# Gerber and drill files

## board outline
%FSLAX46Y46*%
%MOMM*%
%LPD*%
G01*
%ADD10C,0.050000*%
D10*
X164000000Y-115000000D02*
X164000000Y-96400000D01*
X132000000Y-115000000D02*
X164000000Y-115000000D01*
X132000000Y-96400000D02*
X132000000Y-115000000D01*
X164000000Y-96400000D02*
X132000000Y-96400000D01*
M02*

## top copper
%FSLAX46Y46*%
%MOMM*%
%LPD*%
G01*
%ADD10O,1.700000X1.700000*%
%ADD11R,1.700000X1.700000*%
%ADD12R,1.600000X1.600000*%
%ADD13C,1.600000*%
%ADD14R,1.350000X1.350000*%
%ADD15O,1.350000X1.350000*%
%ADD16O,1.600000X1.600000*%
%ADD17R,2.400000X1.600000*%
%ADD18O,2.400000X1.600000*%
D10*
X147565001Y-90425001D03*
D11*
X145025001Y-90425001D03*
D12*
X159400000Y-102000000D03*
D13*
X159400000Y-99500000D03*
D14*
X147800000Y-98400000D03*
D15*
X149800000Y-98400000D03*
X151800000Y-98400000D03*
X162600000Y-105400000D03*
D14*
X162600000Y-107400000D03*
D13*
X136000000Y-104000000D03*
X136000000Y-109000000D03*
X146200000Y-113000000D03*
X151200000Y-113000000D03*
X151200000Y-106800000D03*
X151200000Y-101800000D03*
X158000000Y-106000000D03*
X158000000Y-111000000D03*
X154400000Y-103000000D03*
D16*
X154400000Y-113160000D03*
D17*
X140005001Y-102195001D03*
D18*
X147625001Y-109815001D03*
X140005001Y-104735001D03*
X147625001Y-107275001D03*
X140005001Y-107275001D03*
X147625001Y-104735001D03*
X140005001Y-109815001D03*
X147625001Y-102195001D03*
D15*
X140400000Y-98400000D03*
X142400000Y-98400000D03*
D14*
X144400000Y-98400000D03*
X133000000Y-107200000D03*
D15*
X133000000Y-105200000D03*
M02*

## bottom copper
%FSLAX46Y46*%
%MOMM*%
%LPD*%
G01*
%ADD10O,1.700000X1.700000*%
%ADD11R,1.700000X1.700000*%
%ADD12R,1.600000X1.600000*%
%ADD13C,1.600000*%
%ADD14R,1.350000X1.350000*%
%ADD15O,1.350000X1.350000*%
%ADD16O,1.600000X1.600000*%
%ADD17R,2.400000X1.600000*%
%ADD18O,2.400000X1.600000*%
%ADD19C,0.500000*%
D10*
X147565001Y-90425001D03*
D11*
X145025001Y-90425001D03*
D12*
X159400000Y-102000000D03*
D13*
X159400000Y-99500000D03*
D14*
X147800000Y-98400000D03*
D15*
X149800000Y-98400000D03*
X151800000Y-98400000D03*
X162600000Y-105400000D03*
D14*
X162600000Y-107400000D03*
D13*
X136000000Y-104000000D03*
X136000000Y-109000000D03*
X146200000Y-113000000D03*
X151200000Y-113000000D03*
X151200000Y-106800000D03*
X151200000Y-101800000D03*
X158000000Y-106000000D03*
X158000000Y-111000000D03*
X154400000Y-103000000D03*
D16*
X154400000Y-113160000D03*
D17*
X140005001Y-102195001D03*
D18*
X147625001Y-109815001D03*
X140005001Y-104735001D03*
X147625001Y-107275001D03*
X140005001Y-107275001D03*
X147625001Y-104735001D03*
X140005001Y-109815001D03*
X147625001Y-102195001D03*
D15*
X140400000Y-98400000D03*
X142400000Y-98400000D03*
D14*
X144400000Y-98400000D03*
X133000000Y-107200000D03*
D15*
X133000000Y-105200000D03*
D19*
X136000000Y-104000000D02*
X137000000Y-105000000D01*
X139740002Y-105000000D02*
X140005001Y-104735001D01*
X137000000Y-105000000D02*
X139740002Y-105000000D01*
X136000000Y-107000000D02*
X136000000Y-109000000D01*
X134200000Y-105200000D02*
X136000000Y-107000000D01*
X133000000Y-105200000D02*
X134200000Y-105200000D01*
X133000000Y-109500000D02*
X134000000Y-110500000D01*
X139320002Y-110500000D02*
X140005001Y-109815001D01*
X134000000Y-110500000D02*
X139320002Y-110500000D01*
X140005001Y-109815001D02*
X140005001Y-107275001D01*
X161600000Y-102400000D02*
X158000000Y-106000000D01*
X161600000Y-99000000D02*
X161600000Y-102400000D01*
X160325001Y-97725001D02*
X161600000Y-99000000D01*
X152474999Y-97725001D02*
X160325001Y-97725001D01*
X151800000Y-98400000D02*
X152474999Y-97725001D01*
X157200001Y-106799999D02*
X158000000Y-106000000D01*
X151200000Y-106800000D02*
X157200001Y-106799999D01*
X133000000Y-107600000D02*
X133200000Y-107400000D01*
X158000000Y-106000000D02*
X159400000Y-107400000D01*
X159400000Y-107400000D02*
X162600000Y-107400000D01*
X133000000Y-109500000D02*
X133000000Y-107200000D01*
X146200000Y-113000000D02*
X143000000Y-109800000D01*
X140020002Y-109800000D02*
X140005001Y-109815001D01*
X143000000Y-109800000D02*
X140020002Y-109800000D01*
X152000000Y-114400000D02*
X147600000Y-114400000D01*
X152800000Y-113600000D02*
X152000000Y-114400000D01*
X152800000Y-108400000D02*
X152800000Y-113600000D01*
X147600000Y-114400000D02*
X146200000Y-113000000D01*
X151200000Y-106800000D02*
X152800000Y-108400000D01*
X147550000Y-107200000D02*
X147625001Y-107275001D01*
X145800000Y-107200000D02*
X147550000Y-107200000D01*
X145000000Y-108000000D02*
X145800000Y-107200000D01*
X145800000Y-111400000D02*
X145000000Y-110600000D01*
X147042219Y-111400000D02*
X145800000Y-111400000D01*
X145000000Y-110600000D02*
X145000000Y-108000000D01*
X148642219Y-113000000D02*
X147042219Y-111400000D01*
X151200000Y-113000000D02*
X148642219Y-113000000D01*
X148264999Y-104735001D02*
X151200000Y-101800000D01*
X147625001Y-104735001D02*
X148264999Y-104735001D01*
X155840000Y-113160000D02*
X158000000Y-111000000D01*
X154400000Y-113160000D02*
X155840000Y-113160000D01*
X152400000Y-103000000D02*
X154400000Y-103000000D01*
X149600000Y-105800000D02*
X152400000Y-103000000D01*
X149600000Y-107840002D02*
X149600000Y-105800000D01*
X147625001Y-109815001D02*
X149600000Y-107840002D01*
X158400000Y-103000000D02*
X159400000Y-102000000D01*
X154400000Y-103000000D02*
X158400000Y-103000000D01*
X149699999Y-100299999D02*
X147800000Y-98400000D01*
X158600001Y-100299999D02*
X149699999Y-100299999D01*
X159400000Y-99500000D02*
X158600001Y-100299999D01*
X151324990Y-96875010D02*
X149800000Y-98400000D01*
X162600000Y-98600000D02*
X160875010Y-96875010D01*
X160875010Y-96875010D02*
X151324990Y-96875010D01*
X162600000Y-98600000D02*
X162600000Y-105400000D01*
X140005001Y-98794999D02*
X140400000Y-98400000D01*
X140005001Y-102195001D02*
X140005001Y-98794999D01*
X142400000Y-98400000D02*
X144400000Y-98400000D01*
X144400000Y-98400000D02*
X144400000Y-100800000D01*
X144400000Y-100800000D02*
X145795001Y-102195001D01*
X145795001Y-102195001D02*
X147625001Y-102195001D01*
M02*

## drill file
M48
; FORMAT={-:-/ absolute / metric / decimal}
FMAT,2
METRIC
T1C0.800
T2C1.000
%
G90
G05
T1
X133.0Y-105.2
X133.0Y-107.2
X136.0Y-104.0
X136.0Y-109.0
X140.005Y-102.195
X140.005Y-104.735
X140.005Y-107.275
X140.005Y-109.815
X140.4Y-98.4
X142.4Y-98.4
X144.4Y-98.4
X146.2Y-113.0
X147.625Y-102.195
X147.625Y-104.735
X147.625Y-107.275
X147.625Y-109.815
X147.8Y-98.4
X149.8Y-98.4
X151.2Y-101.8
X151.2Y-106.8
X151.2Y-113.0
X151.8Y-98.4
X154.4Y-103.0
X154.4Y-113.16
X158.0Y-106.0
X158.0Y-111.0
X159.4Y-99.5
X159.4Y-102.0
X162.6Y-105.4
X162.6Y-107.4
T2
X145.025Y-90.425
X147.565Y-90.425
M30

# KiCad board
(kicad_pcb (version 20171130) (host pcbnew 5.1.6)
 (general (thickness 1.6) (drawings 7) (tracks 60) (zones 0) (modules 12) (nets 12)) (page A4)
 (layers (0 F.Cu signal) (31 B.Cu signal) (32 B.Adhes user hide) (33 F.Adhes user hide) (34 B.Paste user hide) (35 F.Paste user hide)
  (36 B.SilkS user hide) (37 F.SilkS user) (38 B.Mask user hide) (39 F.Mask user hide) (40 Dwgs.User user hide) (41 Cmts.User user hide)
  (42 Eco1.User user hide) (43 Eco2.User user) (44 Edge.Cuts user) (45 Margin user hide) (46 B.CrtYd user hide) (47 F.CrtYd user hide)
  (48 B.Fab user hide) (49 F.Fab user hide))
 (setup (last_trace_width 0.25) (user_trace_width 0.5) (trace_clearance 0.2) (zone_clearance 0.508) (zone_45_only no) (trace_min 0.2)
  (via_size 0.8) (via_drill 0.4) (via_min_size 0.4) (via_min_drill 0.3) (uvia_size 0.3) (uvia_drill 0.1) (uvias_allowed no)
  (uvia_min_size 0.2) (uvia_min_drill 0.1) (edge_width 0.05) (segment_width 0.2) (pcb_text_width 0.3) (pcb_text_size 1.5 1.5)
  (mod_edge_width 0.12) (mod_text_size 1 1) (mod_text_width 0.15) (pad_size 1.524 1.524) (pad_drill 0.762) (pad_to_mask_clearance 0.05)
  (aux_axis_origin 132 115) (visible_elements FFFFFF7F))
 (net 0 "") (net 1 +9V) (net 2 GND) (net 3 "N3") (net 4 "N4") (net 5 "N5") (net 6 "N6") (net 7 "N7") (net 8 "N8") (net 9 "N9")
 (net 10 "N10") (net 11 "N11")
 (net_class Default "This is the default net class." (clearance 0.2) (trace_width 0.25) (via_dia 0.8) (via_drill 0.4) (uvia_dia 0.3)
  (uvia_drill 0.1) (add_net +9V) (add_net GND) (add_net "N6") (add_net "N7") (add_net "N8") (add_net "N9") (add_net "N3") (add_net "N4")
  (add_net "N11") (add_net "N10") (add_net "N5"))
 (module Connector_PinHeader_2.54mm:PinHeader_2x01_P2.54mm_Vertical (layer F.Cu) (at 145.025001 90.425001)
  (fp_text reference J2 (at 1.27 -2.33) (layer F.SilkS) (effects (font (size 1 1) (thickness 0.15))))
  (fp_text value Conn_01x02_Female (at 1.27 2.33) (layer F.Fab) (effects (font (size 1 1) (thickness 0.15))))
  (pad 2 thru_hole oval (at 2.54 0) (size 1.7 1.7) (drill 1) (layers *.Cu *.Mask) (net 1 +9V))
  (pad 1 thru_hole rect (at 0 0) (size 1.7 1.7) (drill 1) (layers *.Cu *.Mask) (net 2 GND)))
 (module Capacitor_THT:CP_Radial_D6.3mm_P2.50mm (layer F.Cu) (at 159.4 102 90)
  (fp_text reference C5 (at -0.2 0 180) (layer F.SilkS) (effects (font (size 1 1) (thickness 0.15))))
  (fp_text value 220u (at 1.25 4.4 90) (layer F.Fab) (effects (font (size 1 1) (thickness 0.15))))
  (pad 1 thru_hole rect (at 0 0 90) (size 1.6 1.6) (drill 0.8) (layers *.Cu *.Mask) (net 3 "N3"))
  (pad 2 thru_hole circle (at 2.5 0 90) (size 1.6 1.6) (drill 0.8) (layers *.Cu *.Mask) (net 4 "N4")))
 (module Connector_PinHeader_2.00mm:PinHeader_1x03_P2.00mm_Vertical (layer F.Cu) (at 147.8 98.4 90)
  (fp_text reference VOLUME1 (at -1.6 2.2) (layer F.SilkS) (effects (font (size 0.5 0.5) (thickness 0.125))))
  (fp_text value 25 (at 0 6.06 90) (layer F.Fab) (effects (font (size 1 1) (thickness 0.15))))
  (pad 1 thru_hole rect (at 0 0 90) (size 1.35 1.35) (drill 0.8) (layers *.Cu *.Mask) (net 4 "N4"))
  (pad 2 thru_hole oval (at 0 2 90) (size 1.35 1.35) (drill 0.8) (layers *.Cu *.Mask) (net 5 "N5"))
  (pad 3 thru_hole oval (at 0 4 90) (size 1.35 1.35) (drill 0.8) (layers *.Cu *.Mask) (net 2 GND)))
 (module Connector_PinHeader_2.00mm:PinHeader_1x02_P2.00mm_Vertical (layer F.Cu) (at 162.6 107.4 180)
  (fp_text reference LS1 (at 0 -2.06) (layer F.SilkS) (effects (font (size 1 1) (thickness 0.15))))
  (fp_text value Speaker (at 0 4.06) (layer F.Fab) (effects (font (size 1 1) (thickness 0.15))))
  (pad 2 thru_hole oval (at 0 2 180) (size 1.35 1.35) (drill 0.8) (layers *.Cu *.Mask) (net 5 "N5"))
  (pad 1 thru_hole rect (at 0 0 180) (size 1.35 1.35) (drill 0.8) (layers *.Cu *.Mask) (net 2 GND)))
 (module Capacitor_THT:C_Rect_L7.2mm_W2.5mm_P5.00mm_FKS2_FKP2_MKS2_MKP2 (layer F.Cu) (at 136 104 270)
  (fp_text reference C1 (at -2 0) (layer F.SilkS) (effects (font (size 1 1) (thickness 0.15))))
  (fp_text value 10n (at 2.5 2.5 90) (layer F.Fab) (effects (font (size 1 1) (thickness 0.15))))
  (pad 1 thru_hole circle (at 0 0 270) (size 1.6 1.6) (drill 0.8) (layers *.Cu *.Mask) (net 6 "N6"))
  (pad 2 thru_hole circle (at 5 0 270) (size 1.6 1.6) (drill 0.8) (layers *.Cu *.Mask) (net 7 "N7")))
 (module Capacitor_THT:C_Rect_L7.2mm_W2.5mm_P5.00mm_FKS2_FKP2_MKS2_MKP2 (layer F.Cu) (at 151.2 113 180)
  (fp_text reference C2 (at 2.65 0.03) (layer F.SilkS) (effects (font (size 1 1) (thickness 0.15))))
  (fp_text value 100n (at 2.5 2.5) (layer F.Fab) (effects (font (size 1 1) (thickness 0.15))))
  (pad 2 thru_hole circle (at 5 0 180) (size 1.6 1.6) (drill 0.8) (layers *.Cu *.Mask) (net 2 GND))
  (pad 1 thru_hole circle (at 0 0 180) (size 1.6 1.6) (drill 0.8) (layers *.Cu *.Mask) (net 1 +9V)))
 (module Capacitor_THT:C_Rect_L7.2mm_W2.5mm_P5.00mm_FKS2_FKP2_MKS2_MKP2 (layer F.Cu) (at 151.2 106.8 90)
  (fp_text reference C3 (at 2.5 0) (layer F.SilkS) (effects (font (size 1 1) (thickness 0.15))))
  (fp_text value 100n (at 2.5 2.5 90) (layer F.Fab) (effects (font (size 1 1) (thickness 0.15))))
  (pad 1 thru_hole circle (at 0 0 90) (size 1.6 1.6) (drill 0.8) (layers *.Cu *.Mask) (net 2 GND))
  (pad 2 thru_hole circle (at 5 0 90) (size 1.6 1.6) (drill 0.8) (layers *.Cu *.Mask) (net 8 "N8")))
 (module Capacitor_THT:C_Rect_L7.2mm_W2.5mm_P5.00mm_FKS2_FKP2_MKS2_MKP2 (layer F.Cu) (at 158 111 90)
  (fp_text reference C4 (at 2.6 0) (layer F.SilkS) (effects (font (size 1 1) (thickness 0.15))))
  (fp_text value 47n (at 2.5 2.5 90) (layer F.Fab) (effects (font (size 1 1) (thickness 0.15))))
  (pad 2 thru_hole circle (at 5 0 90) (size 1.6 1.6) (drill 0.8) (layers *.Cu *.Mask) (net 2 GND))
  (pad 1 thru_hole circle (at 0 0 90) (size 1.6 1.6) (drill 0.8) (layers *.Cu *.Mask) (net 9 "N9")))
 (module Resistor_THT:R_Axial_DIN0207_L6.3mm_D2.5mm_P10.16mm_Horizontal (layer F.Cu) (at 154.4 103 270)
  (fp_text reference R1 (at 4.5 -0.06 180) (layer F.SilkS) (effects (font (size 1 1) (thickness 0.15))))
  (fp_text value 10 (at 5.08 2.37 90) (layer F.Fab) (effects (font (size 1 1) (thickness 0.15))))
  (pad 1 thru_hole circle (at 0 0 270) (size 1.6 1.6) (drill 0.8) (layers *.Cu *.Mask) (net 3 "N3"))
  (pad 2 thru_hole oval (at 10.16 0 270) (size 1.6 1.6) (drill 0.8) (layers *.Cu *.Mask) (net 9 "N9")))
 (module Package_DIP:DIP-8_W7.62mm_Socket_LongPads (layer F.Cu) (at 140.005001 102.195001)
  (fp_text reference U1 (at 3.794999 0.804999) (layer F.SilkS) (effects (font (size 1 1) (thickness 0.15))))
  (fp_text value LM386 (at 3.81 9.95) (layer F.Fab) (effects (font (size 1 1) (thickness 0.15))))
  (pad 1 thru_hole rect (at 0 0) (size 2.4 1.6) (drill 0.8) (layers *.Cu *.Mask) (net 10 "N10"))
  (pad 5 thru_hole oval (at 7.62 7.62) (size 2.4 1.6) (drill 0.8) (layers *.Cu *.Mask) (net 3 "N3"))
  (pad 2 thru_hole oval (at 0 2.54) (size 2.4 1.6) (drill 0.8) (layers *.Cu *.Mask) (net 6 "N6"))
  (pad 6 thru_hole oval (at 7.62 5.08) (size 2.4 1.6) (drill 0.8) (layers *.Cu *.Mask) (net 1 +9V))
  (pad 3 thru_hole oval (at 0 5.08) (size 2.4 1.6) (drill 0.8) (layers *.Cu *.Mask) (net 2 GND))
  (pad 7 thru_hole oval (at 7.62 2.54) (size 2.4 1.6) (drill 0.8) (layers *.Cu *.Mask) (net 8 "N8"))
  (pad 4 thru_hole oval (at 0 7.62) (size 2.4 1.6) (drill 0.8) (layers *.Cu *.Mask) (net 2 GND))
  (pad 8 thru_hole oval (at 7.62 0) (size 2.4 1.6) (drill 0.8) (layers *.Cu *.Mask) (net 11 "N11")))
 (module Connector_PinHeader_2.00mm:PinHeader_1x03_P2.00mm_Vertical (layer F.Cu) (at 144.4 98.4 270)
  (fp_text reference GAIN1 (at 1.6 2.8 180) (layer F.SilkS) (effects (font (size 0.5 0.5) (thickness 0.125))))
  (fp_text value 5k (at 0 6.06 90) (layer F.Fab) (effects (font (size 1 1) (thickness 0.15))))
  (pad 3 thru_hole oval (at 0 4 270) (size 1.35 1.35) (drill 0.8) (layers *.Cu *.Mask) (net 10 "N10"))
  (pad 2 thru_hole oval (at 0 2 270) (size 1.35 1.35) (drill 0.8) (layers *.Cu *.Mask) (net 11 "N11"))
  (pad 1 thru_hole rect (at 0 0 270) (size 1.35 1.35) (drill 0.8) (layers *.Cu *.Mask) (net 11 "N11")))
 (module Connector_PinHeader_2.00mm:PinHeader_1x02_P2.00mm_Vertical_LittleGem (layer F.Cu) (at 133 107.2 180)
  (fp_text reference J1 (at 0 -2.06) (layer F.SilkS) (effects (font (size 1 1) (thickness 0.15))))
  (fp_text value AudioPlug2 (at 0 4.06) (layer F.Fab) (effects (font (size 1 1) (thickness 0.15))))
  (pad S thru_hole rect (at 0 0 180) (size 1.35 1.35) (drill 0.8) (layers *.Cu *.Mask) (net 2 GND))
  (pad T thru_hole oval (at 0 2 180) (size 1.35 1.35) (drill 0.8) (layers *.Cu *.Mask) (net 7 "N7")))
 (gr_line (start 164 115) (end 164 96.4) (layer Edge.Cuts) (width 0.05))
 (gr_line (start 132 115) (end 164 115) (layer Edge.Cuts) (width 0.05))
 (gr_line (start 132 96.4) (end 132 115) (layer Edge.Cuts) (width 0.05))
 (gr_line (start 164 96.4) (end 132 96.4) (layer Edge.Cuts) (width 0.05))
 (segment (start 136 104) (end 137 105) (width 0.5) (layer B.Cu) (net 6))
 (segment (start 139.740002 105) (end 140.005001 104.735001) (width 0.5) (layer B.Cu) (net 6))
 (segment (start 137 105) (end 139.740002 105) (width 0.5) (layer B.Cu) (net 6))
 (segment (start 136 107) (end 136 109) (width 0.5) (layer B.Cu) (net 7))
 (segment (start 134.2 105.2) (end 136 107) (width 0.5) (layer B.Cu) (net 7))
 (segment (start 133 105.2) (end 134.2 105.2) (width 0.5) (layer B.Cu) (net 7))
 (segment (start 133 109.5) (end 134 110.5) (width 0.5) (layer B.Cu) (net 2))
 (segment (start 139.320002 110.5) (end 140.005001 109.815001) (width 0.5) (layer B.Cu) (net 2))
 (segment (start 134 110.5) (end 139.320002 110.5) (width 0.5) (layer B.Cu) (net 2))
 (segment (start 140.005001 109.815001) (end 140.005001 107.275001) (width 0.5) (layer B.Cu) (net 2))
 (segment (start 161.6 102.4) (end 158 106) (width 0.5) (layer B.Cu) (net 2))
 (segment (start 161.6 99) (end 161.6 102.4) (width 0.5) (layer B.Cu) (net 2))
 (segment (start 160.325001 97.725001) (end 161.6 99) (width 0.5) (layer B.Cu) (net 2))
 (segment (start 152.474999 97.725001) (end 160.325001 97.725001) (width 0.5) (layer B.Cu) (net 2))
 (segment (start 151.8 98.4) (end 152.474999 97.725001) (width 0.5) (layer B.Cu) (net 2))
 (segment (start 157.200001 106.799999) (end 158 106) (width 0.5) (layer B.Cu) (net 2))
 (segment (start 151.2 106.8) (end 157.200001 106.799999) (width 0.5) (layer B.Cu) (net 2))
 (segment (start 133 107.6) (end 133.2 107.4) (width 0.5) (layer B.Cu) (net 2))
 (segment (start 158 106) (end 159.4 107.4) (width 0.5) (layer B.Cu) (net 2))
 (segment (start 159.4 107.4) (end 162.6 107.4) (width 0.5) (layer B.Cu) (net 2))
 (segment (start 133 109.5) (end 133 107.2) (width 0.5) (layer B.Cu) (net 2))
 (segment (start 146.2 113) (end 143 109.8) (width 0.5) (layer B.Cu) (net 2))
 (segment (start 140.020002 109.8) (end 140.005001 109.815001) (width 0.5) (layer B.Cu) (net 2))
 (segment (start 143 109.8) (end 140.020002 109.8) (width 0.5) (layer B.Cu) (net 2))
 (segment (start 152 114.4) (end 147.6 114.4) (width 0.5) (layer B.Cu) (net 2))
 (segment (start 152.8 113.6) (end 152 114.4) (width 0.5) (layer B.Cu) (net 2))
 (segment (start 152.8 108.4) (end 152.8 113.6) (width 0.5) (layer B.Cu) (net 2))
 (segment (start 147.6 114.4) (end 146.2 113) (width 0.5) (layer B.Cu) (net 2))
 (segment (start 151.2 106.8) (end 152.8 108.4) (width 0.5) (layer B.Cu) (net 2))
 (segment (start 147.55 107.2) (end 147.625001 107.275001) (width 0.5) (layer B.Cu) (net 1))
 (segment (start 145.8 107.2) (end 147.55 107.2) (width 0.5) (layer B.Cu) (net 1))
 (segment (start 145 108) (end 145.8 107.2) (width 0.5) (layer B.Cu) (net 1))
 (segment (start 145.8 111.4) (end 145 110.6) (width 0.5) (layer B.Cu) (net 1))
 (segment (start 147.042219 111.4) (end 145.8 111.4) (width 0.5) (layer B.Cu) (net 1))
 (segment (start 145 110.6) (end 145 108) (width 0.5) (layer B.Cu) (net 1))
 (segment (start 148.642219 113) (end 147.042219 111.4) (width 0.5) (layer B.Cu) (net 1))
 (segment (start 151.2 113) (end 148.642219 113) (width 0.5) (layer B.Cu) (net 1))
 (segment (start 148.264999 104.735001) (end 151.2 101.8) (width 0.5) (layer B.Cu) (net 8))
 (segment (start 147.625001 104.735001) (end 148.264999 104.735001) (width 0.5) (layer B.Cu) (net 8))
 (segment (start 155.84 113.16) (end 158 111) (width 0.5) (layer B.Cu) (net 9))
 (segment (start 154.4 113.16) (end 155.84 113.16) (width 0.5) (layer B.Cu) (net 9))
 (segment (start 152.4 103) (end 154.4 103) (width 0.5) (layer B.Cu) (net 3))
 (segment (start 149.6 105.8) (end 152.4 103) (width 0.5) (layer B.Cu) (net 3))
 (segment (start 149.6 107.840002) (end 149.6 105.8) (width 0.5) (layer B.Cu) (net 3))
 (segment (start 147.625001 109.815001) (end 149.6 107.840002) (width 0.5) (layer B.Cu) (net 3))
 (segment (start 158.4 103) (end 159.4 102) (width 0.5) (layer B.Cu) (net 3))
 (segment (start 154.4 103) (end 158.4 103) (width 0.5) (layer B.Cu) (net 3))
 (segment (start 149.699999 100.299999) (end 147.8 98.4) (width 0.5) (layer B.Cu) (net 4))
 (segment (start 158.600001 100.299999) (end 149.699999 100.299999) (width 0.5) (layer B.Cu) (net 4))
 (segment (start 159.4 99.5) (end 158.600001 100.299999) (width 0.5) (layer B.Cu) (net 4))
 (segment (start 151.32499 96.87501) (end 149.8 98.4) (width 0.5) (layer B.Cu) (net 5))
 (segment (start 162.6 98.6) (end 160.87501 96.87501) (width 0.5) (layer B.Cu) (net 5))
 (segment (start 160.87501 96.87501) (end 151.32499 96.87501) (width 0.5) (layer B.Cu) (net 5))
 (segment (start 162.6 98.6) (end 162.6 105.4) (width 0.5) (layer B.Cu) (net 5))
 (segment (start 140.005001 98.794999) (end 140.4 98.4) (width 0.5) (layer B.Cu) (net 10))
 (segment (start 140.005001 102.195001) (end 140.005001 98.794999) (width 0.5) (layer B.Cu) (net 10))
 (segment (start 142.4 98.4) (end 144.4 98.4) (width 0.5) (layer B.Cu) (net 11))
 (segment (start 144.4 98.4) (end 144.4 100.8) (width 0.5) (layer B.Cu) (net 11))
 (segment (start 144.4 100.8) (end 145.795001 102.195001) (width 0.5) (layer B.Cu) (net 11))
 (segment (start 145.795001 102.195001) (end 147.625001 102.195001) (width 0.5) (layer B.Cu) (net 11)))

